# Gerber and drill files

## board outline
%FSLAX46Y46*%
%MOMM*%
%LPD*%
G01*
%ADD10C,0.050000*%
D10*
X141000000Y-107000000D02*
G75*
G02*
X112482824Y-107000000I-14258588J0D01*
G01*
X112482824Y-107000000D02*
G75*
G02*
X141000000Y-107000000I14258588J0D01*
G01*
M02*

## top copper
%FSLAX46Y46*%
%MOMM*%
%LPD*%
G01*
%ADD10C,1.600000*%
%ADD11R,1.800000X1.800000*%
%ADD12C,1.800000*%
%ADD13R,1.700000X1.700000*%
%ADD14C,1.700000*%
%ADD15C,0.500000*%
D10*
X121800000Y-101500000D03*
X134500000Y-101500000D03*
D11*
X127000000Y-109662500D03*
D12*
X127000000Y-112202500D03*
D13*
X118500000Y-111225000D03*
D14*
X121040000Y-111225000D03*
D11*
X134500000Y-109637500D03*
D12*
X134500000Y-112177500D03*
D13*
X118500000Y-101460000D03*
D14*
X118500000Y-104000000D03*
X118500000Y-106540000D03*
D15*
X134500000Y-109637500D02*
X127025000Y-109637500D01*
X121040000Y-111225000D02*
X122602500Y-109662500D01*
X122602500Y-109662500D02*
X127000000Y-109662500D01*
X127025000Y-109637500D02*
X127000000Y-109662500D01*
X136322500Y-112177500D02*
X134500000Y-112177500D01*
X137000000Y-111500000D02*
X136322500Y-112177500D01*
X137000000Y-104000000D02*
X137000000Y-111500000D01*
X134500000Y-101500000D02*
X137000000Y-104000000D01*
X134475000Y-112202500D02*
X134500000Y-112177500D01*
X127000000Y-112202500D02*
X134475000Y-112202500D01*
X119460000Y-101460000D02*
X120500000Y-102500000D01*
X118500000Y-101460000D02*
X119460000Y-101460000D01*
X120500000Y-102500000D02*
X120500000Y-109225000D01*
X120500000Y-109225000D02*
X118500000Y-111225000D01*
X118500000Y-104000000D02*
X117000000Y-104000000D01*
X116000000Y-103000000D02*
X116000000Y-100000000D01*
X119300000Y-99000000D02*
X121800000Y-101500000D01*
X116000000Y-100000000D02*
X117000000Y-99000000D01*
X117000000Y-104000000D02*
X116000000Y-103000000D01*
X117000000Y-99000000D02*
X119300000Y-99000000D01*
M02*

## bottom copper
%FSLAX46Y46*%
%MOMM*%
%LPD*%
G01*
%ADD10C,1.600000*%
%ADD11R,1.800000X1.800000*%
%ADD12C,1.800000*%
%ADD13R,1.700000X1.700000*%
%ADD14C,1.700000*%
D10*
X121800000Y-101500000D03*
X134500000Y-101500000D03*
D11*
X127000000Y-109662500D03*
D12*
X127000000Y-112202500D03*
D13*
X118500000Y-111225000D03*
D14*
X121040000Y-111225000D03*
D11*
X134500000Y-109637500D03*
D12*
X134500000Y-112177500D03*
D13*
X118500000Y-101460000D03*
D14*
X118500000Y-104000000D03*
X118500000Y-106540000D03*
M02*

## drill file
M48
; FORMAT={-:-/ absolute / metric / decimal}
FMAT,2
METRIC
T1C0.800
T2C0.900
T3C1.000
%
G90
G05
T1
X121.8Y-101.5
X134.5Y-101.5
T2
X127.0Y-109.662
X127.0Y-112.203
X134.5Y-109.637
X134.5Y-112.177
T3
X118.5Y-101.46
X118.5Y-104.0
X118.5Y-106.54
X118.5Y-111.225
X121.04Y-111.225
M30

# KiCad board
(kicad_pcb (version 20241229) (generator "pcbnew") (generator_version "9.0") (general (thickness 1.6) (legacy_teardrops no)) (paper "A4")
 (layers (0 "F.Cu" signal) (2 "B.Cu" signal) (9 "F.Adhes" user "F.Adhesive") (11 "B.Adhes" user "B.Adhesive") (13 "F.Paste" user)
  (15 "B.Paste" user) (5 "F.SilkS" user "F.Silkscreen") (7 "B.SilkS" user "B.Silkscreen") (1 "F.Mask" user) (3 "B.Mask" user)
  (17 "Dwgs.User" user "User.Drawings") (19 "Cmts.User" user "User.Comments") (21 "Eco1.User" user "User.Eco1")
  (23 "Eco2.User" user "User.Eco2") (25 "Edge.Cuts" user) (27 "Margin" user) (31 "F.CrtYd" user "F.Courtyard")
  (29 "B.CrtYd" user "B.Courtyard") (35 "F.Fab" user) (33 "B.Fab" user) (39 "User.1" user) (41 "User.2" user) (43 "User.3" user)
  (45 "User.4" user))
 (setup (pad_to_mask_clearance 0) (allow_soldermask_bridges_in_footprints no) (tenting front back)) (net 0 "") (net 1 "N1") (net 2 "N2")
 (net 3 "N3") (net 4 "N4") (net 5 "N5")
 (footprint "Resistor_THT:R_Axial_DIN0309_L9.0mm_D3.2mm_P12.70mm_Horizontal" (layer "F.Cu") (at 121.8 101.5)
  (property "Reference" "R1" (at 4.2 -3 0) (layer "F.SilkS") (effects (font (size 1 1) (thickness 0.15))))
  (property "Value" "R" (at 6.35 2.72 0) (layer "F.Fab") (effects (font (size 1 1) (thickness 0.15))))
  (pad "1" thru_hole circle (at 0 0) (size 1.6 1.6) (drill 0.8) (layers "*.Cu" "*.Mask") (remove_unused_layers no) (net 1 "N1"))
  (pad "2" thru_hole circle (at 12.7 0) (size 1.6 1.6) (drill 0.8) (layers "*.Cu" "*.Mask") (remove_unused_layers no) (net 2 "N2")))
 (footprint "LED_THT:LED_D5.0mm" (layer "F.Cu") (at 127 109.6625 -90)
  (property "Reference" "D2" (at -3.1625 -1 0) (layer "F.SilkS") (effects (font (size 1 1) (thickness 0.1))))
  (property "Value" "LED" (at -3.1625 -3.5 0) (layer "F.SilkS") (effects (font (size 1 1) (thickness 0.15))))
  (pad "1" thru_hole rect (at 0 0 270) (size 1.8 1.8) (drill 0.9) (layers "*.Cu" "*.Mask") (remove_unused_layers no) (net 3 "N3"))
  (pad "2" thru_hole circle (at 2.54 0 270) (size 1.8 1.8) (drill 0.9) (layers "*.Cu" "*.Mask") (remove_unused_layers no) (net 2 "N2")))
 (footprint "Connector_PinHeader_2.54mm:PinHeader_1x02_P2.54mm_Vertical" (layer "F.Cu") (at 118.5 111.225 90)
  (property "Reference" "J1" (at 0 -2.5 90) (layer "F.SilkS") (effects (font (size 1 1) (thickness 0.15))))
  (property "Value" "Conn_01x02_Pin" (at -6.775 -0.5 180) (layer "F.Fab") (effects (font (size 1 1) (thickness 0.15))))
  (pad "1" thru_hole rect (at 0 0 90) (size 1.7 1.7) (drill 1) (layers "*.Cu" "*.Mask") (remove_unused_layers no) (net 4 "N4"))
  (pad "2" thru_hole circle (at 0 2.54 90) (size 1.7 1.7) (drill 1) (layers "*.Cu" "*.Mask") (remove_unused_layers no) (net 3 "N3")))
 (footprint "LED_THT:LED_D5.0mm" (layer "F.Cu") (at 134.5 109.6375 -90)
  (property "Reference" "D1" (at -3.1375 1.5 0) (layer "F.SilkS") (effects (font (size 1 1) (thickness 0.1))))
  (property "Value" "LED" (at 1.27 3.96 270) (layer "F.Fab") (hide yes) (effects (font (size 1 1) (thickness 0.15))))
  (pad "1" thru_hole rect (at 0 0 270) (size 1.8 1.8) (drill 0.9) (layers "*.Cu" "*.Mask") (remove_unused_layers no) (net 3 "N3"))
  (pad "2" thru_hole circle (at 2.54 0 270) (size 1.8 1.8) (drill 0.9) (layers "*.Cu" "*.Mask") (remove_unused_layers no) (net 2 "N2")))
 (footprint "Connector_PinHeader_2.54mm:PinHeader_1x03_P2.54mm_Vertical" (layer "F.Cu") (at 118.5 101.46)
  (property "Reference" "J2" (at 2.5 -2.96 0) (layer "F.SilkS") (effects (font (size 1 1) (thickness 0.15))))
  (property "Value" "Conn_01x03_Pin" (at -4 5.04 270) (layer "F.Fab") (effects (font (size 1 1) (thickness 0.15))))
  (pad "1" thru_hole rect (at 0 0) (size 1.7 1.7) (drill 1) (layers "*.Cu" "*.Mask") (remove_unused_layers no) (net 4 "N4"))
  (pad "2" thru_hole circle (at 0 2.54) (size 1.7 1.7) (drill 1) (layers "*.Cu" "*.Mask") (remove_unused_layers no) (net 1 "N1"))
  (pad "3" thru_hole circle (at 0 5.08) (size 1.7 1.7) (drill 1) (layers "*.Cu" "*.Mask") (remove_unused_layers no) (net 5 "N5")))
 (gr_circle (center 126.741412 107) (end 139.676145 113) (stroke (width 0.05) (type default)) (fill no) (layer "Edge.Cuts"))
 (segment (start 134.5 109.6375) (end 127.025 109.6375) (width 0.5) (layer "F.Cu") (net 3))
 (segment (start 121.04 111.225) (end 122.6025 109.6625) (width 0.5) (layer "F.Cu") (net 3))
 (segment (start 122.6025 109.6625) (end 127 109.6625) (width 0.5) (layer "F.Cu") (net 3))
 (segment (start 127.025 109.6375) (end 127 109.6625) (width 0.5) (layer "F.Cu") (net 3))
 (segment (start 136.3225 112.1775) (end 134.5 112.1775) (width 0.5) (layer "F.Cu") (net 2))
 (segment (start 137 111.5) (end 136.3225 112.1775) (width 0.5) (layer "F.Cu") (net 2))
 (segment (start 137 104) (end 137 111.5) (width 0.5) (layer "F.Cu") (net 2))
 (segment (start 134.5 101.5) (end 137 104) (width 0.5) (layer "F.Cu") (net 2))
 (segment (start 134.475 112.2025) (end 134.5 112.1775) (width 0.5) (layer "F.Cu") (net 2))
 (segment (start 127 112.2025) (end 134.475 112.2025) (width 0.5) (layer "F.Cu") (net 2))
 (segment (start 119.46 101.46) (end 120.5 102.5) (width 0.5) (layer "F.Cu") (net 4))
 (segment (start 118.5 101.46) (end 119.46 101.46) (width 0.5) (layer "F.Cu") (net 4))
 (segment (start 120.5 102.5) (end 120.5 109.225) (width 0.5) (layer "F.Cu") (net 4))
 (segment (start 120.5 109.225) (end 118.5 111.225) (width 0.5) (layer "F.Cu") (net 4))
 (segment (start 118.5 104) (end 117 104) (width 0.5) (layer "F.Cu") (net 1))
 (segment (start 116 103) (end 116 100) (width 0.5) (layer "F.Cu") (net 1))
 (segment (start 119.3 99) (end 121.8 101.5) (width 0.5) (layer "F.Cu") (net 1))
 (segment (start 116 100) (end 117 99) (width 0.5) (layer "F.Cu") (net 1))
 (segment (start 117 104) (end 116 103) (width 0.5) (layer "F.Cu") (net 1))
 (segment (start 117 99) (end 119.3 99) (width 0.5) (layer "F.Cu") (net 1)))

